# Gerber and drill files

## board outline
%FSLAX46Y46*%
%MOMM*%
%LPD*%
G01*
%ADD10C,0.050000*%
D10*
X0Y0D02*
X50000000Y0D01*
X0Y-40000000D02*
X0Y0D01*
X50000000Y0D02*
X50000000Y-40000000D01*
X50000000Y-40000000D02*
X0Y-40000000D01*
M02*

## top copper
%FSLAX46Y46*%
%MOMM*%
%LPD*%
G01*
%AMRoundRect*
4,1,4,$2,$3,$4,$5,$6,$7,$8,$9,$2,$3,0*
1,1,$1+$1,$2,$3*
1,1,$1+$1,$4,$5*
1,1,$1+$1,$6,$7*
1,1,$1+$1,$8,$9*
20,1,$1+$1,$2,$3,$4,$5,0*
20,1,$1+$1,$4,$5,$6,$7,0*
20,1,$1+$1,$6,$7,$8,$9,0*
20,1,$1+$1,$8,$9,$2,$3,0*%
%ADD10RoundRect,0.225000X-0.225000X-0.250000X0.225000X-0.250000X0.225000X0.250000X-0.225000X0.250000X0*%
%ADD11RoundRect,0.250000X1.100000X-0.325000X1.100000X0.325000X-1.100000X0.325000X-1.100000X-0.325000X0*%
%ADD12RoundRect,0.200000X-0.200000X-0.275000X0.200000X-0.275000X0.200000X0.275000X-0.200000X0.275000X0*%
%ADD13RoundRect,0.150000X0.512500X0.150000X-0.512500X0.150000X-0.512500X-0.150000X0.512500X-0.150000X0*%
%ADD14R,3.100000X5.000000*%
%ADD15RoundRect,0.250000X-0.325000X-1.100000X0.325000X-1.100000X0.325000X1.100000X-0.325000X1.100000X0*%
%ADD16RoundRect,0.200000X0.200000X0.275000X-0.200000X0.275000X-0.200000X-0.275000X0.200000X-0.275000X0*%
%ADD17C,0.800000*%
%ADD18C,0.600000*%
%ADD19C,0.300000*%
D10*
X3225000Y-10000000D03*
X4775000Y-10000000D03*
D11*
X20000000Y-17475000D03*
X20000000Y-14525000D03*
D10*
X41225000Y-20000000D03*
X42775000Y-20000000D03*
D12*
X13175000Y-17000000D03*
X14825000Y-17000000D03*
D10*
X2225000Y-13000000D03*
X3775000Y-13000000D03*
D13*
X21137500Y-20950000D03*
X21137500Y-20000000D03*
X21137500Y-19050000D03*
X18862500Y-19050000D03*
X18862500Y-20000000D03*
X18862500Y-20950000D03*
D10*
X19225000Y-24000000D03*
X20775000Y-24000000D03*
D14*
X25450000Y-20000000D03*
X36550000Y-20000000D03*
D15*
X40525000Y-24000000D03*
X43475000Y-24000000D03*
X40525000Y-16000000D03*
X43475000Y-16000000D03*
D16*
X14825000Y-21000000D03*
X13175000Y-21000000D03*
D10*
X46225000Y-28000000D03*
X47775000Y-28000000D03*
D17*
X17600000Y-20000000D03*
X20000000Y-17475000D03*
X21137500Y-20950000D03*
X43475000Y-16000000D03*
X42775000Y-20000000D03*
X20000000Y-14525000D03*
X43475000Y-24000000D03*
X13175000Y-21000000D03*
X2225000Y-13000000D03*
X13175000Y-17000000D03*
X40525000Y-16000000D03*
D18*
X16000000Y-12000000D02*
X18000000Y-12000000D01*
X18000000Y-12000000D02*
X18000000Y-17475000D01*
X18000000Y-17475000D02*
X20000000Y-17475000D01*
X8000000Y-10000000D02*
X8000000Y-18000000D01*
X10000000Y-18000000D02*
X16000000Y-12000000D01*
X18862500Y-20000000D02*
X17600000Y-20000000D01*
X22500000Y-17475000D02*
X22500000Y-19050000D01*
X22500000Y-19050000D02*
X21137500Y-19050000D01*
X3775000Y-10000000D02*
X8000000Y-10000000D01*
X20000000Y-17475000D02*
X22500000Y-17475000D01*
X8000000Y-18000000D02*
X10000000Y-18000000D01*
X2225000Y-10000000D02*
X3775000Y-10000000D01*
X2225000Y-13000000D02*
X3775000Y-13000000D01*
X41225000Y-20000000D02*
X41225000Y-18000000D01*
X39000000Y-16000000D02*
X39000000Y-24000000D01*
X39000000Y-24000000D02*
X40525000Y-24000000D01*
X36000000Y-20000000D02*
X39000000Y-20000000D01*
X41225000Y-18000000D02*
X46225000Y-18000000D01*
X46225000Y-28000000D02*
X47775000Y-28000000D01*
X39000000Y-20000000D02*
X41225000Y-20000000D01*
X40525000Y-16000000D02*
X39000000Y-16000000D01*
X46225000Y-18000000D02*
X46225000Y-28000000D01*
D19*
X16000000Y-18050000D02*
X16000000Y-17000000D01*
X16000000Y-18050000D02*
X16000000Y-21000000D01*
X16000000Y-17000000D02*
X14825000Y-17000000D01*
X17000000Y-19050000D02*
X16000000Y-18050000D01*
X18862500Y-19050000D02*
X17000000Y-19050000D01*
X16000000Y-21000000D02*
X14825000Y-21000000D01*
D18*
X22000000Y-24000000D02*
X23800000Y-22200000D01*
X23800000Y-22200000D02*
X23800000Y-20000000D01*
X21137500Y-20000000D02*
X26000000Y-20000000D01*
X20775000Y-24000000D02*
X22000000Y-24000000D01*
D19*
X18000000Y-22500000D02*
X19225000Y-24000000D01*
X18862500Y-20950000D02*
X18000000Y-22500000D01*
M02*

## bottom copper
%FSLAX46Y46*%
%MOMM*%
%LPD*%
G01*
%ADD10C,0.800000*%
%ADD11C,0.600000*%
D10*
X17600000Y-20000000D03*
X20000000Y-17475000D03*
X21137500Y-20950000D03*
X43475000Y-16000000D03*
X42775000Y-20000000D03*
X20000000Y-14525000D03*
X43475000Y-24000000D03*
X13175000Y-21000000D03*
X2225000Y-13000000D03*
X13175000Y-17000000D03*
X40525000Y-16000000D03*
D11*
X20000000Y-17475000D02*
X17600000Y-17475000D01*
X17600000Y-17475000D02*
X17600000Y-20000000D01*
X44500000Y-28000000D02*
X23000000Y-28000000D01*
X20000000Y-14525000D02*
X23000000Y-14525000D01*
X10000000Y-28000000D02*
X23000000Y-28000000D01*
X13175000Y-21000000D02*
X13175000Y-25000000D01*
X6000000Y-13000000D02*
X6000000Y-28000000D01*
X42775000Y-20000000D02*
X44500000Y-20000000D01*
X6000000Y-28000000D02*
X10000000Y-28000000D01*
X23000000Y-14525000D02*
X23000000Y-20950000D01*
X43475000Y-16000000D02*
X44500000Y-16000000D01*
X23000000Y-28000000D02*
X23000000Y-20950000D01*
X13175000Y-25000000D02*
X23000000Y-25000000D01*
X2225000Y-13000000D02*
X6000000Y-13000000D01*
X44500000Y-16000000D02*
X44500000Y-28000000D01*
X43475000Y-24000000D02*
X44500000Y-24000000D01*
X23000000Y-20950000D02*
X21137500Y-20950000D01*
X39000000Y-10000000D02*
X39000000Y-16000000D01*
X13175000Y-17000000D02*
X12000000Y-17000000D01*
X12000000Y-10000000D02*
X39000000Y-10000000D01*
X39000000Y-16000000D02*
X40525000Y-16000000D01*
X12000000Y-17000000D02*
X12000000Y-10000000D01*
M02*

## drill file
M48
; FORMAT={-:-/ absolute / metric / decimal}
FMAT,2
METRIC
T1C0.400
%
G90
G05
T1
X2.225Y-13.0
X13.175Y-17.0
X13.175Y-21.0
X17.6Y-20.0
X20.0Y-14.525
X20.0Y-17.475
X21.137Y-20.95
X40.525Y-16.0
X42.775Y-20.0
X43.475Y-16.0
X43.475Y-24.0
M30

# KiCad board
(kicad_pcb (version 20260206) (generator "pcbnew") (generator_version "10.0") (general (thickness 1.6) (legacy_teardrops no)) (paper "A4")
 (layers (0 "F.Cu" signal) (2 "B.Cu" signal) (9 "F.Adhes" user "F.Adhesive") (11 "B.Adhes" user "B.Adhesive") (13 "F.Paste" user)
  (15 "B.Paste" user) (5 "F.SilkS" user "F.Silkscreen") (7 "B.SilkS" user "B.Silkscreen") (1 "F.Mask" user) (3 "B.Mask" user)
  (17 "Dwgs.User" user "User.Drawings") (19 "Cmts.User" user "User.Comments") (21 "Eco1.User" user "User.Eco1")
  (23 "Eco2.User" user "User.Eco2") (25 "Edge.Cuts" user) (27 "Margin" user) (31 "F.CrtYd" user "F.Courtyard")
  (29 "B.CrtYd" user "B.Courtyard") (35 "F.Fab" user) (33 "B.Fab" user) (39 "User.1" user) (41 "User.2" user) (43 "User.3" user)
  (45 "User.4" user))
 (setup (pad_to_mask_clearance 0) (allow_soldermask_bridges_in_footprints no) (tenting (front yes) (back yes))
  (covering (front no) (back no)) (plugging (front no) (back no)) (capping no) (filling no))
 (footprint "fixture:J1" (layer "F.Cu") (at 4 10)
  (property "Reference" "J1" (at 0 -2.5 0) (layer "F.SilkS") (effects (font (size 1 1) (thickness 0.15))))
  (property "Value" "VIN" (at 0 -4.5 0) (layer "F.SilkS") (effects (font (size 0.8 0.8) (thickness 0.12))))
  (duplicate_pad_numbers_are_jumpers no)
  (pad "1" smd roundrect (at -0.775 0) (size 0.9 0.95) (layers "F.Cu" "F.Mask" "F.Paste") (roundrect_rratio 0.25) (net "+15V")
   (thermal_bridge_angle 45))
  (pad "2" smd roundrect (at 0.775 0) (size 0.9 0.95) (layers "F.Cu" "F.Mask" "F.Paste") (roundrect_rratio 0.25) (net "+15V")
   (thermal_bridge_angle 45)))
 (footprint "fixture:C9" (layer "F.Cu") (at 20 16 90)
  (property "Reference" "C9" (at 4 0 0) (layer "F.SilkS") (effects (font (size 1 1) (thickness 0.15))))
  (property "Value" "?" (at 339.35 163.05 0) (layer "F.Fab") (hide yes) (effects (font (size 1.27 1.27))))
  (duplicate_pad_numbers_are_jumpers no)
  (pad "1" smd roundrect (at -1.475 0 90) (size 1.15 2.7) (layers "F.Cu" "F.Mask" "F.Paste") (roundrect_rratio 0.217391) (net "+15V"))
  (pad "2" smd roundrect (at 1.475 0 90) (size 1.15 2.7) (layers "F.Cu" "F.Mask" "F.Paste") (roundrect_rratio 0.217391) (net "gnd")))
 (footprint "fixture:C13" (layer "F.Cu") (at 42 20)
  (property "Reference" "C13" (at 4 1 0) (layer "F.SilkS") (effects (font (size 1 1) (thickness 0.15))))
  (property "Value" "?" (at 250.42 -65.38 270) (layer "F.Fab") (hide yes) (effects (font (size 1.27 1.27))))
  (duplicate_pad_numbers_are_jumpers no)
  (pad "1" smd roundrect (at -0.775 0) (size 0.9 0.95) (layers "F.Cu" "F.Mask" "F.Paste") (roundrect_rratio 0.25) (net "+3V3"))
  (pad "2" smd roundrect (at 0.775 0) (size 0.9 0.95) (layers "F.Cu" "F.Mask" "F.Paste") (roundrect_rratio 0.25) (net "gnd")))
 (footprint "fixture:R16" (layer "F.Cu") (at 14 17)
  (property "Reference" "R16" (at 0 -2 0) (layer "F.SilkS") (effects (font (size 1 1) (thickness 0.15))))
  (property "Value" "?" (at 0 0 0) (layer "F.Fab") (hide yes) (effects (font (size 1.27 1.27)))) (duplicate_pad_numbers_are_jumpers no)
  (pad "1" smd roundrect (at -0.825 0) (size 0.8 0.95) (layers "F.Cu" "F.Mask" "F.Paste") (roundrect_rratio 0.25) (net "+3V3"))
  (pad "2" smd roundrect (at 0.825 0) (size 0.8 0.95) (layers "F.Cu" "F.Mask" "F.Paste") (roundrect_rratio 0.25) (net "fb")))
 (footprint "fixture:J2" (layer "F.Cu") (at 3 13)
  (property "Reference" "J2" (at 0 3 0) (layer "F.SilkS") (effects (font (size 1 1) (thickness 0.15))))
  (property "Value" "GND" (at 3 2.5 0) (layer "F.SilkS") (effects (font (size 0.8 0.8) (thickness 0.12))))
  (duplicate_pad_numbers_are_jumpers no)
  (pad "1" smd roundrect (at -0.775 0) (size 0.9 0.95) (layers "F.Cu" "F.Mask" "F.Paste") (roundrect_rratio 0.25) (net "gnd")
   (thermal_bridge_angle 45))
  (pad "2" smd roundrect (at 0.775 0) (size 0.9 0.95) (layers "F.Cu" "F.Mask" "F.Paste") (roundrect_rratio 0.25) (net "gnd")
   (thermal_bridge_angle 45)))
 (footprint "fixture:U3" (layer "F.Cu") (at 20 20 180)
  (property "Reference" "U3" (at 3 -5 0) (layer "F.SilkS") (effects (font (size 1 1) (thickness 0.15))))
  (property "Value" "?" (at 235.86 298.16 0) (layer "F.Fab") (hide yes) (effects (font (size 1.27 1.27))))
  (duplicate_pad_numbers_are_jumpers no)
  (pad "1" smd roundrect (at -1.1375 -0.95 180) (size 1.325 0.6) (layers "F.Cu" "F.Mask" "F.Paste") (roundrect_rratio 0.25) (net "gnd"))
  (pad "2" smd roundrect (at -1.1375 0 180) (size 1.325 0.6) (layers "F.Cu" "F.Mask" "F.Paste") (roundrect_rratio 0.25) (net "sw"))
  (pad "3" smd roundrect (at -1.1375 0.95 180) (size 1.325 0.6) (layers "F.Cu" "F.Mask" "F.Paste") (roundrect_rratio 0.25) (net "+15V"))
  (pad "4" smd roundrect (at 1.1375 0.95 180) (size 1.325 0.6) (layers "F.Cu" "F.Mask" "F.Paste") (roundrect_rratio 0.25) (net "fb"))
  (pad "5" smd roundrect (at 1.1375 0 180) (size 1.325 0.6) (layers "F.Cu" "F.Mask" "F.Paste") (roundrect_rratio 0.25) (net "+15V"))
  (pad "6" smd roundrect (at 1.1375 -0.95 180) (size 1.325 0.6) (layers "F.Cu" "F.Mask" "F.Paste") (roundrect_rratio 0.25) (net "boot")))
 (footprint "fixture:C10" (layer "F.Cu") (at 20 24)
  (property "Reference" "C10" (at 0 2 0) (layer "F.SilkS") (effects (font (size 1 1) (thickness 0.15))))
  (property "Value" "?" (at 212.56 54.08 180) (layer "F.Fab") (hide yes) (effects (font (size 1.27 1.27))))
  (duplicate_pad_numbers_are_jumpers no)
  (pad "1" smd roundrect (at -0.775 0) (size 0.9 0.95) (layers "F.Cu" "F.Mask" "F.Paste") (roundrect_rratio 0.25) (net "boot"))
  (pad "2" smd roundrect (at 0.775 0) (size 0.9 0.95) (layers "F.Cu" "F.Mask" "F.Paste") (roundrect_rratio 0.25) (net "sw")))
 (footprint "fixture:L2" (layer "F.Cu") (at 31 20)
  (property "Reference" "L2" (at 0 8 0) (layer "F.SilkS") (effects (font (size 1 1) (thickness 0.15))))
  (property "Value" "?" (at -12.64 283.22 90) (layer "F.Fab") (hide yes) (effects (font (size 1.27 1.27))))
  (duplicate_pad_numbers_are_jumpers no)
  (pad "1" smd rect (at -5.55 0) (size 3.1 5) (layers "F.Cu" "F.Mask" "F.Paste") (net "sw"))
  (pad "2" smd rect (at 5.55 0) (size 3.1 5) (layers "F.Cu" "F.Mask" "F.Paste") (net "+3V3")))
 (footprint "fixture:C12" (layer "F.Cu") (at 42 24)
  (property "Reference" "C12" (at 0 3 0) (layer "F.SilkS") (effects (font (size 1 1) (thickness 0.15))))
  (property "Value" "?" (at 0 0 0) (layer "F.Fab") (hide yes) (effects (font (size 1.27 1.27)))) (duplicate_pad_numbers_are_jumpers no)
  (pad "1" smd roundrect (at -1.475 0) (size 1.15 2.7) (layers "F.Cu" "F.Mask" "F.Paste") (roundrect_rratio 0.217391) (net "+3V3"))
  (pad "2" smd roundrect (at 1.475 0) (size 1.15 2.7) (layers "F.Cu" "F.Mask" "F.Paste") (roundrect_rratio 0.217391) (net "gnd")))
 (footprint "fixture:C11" (layer "F.Cu") (at 42 16)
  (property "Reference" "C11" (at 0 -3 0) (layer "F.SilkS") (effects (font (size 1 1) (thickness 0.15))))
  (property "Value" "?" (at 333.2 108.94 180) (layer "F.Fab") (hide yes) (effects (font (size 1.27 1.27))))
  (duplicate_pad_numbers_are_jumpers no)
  (pad "1" smd roundrect (at -1.475 0) (size 1.15 2.7) (layers "F.Cu" "F.Mask" "F.Paste") (roundrect_rratio 0.217391) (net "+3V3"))
  (pad "2" smd roundrect (at 1.475 0) (size 1.15 2.7) (layers "F.Cu" "F.Mask" "F.Paste") (roundrect_rratio 0.217391) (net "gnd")))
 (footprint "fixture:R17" (layer "F.Cu") (at 14 21 180)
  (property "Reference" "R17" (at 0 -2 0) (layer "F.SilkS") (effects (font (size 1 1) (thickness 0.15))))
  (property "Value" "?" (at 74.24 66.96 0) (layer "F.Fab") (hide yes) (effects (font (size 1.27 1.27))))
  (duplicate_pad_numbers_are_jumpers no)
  (pad "1" smd roundrect (at -0.825 0 180) (size 0.8 0.95) (layers "F.Cu" "F.Mask" "F.Paste") (roundrect_rratio 0.25) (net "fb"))
  (pad "2" smd roundrect (at 0.825 0 180) (size 0.8 0.95) (layers "F.Cu" "F.Mask" "F.Paste") (roundrect_rratio 0.25) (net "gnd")))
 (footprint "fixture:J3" (layer "F.Cu") (at 47 28)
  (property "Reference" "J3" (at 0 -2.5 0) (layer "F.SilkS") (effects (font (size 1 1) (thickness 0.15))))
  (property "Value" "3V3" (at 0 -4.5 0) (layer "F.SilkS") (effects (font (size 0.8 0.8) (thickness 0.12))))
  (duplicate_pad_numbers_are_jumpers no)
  (pad "1" smd roundrect (at -0.775 0) (size 0.9 0.95) (layers "F.Cu" "F.Mask" "F.Paste") (roundrect_rratio 0.25) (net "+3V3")
   (thermal_bridge_angle 45))
  (pad "2" smd roundrect (at 0.775 0) (size 0.9 0.95) (layers "F.Cu" "F.Mask" "F.Paste") (roundrect_rratio 0.25) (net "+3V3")
   (thermal_bridge_angle 45)))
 (gr_line (start 0 0) (end 50 0) (stroke (width 0.05) (type default)) (layer "Edge.Cuts"))
 (gr_line (start 0 40) (end 0 0) (stroke (width 0.05) (type default)) (layer "Edge.Cuts"))
 (gr_line (start 50 0) (end 50 40) (stroke (width 0.05) (type default)) (layer "Edge.Cuts"))
 (gr_line (start 50 40) (end 0 40) (stroke (width 0.05) (type default)) (layer "Edge.Cuts"))
 (segment (start 16 12) (end 18 12) (width 0.6) (layer "F.Cu") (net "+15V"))
 (segment (start 18 12) (end 18 17.475) (width 0.6) (layer "F.Cu") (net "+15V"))
 (segment (start 18 17.475) (end 20 17.475) (width 0.6) (layer "F.Cu") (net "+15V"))
 (segment (start 8 10) (end 8 18) (width 0.6) (layer "F.Cu") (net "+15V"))
 (segment (start 10 18) (end 16 12) (width 0.6) (layer "F.Cu") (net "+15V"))
 (segment (start 18.8625 20) (end 17.6 20) (width 0.6) (layer "F.Cu") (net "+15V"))
 (segment (start 22.5 17.475) (end 22.5 19.05) (width 0.6) (layer "F.Cu") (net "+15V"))
 (segment (start 22.5 19.05) (end 21.1375 19.05) (width 0.6) (layer "F.Cu") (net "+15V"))
 (segment (start 3.775 10) (end 8 10) (width 0.6) (layer "F.Cu") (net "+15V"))
 (segment (start 20 17.475) (end 22.5 17.475) (width 0.6) (layer "F.Cu") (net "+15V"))
 (segment (start 8 18) (end 10 18) (width 0.6) (layer "F.Cu") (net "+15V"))
 (segment (start 2.225 10) (end 3.775 10) (width 0.6) (layer "F.Cu") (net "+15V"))
 (via (at 17.6 20) (size 0.8) (drill 0.4) (layers "F.Cu" "B.Cu") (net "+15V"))
 (via (at 20 17.475) (size 0.8) (drill 0.4) (layers "F.Cu" "B.Cu") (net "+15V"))
 (segment (start 20 17.475) (end 17.6 17.475) (width 0.6) (layer "B.Cu") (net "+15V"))
 (segment (start 17.6 17.475) (end 17.6 20) (width 0.6) (layer "B.Cu") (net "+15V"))
 (segment (start 2.225 13) (end 3.775 13) (width 0.6) (layer "F.Cu") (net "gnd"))
 (via (at 21.1375 20.95) (size 0.8) (drill 0.4) (layers "F.Cu" "B.Cu") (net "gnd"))
 (via (at 43.475 16) (size 0.8) (drill 0.4) (layers "F.Cu" "B.Cu") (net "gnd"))
 (via (at 42.775 20) (size 0.8) (drill 0.4) (layers "F.Cu" "B.Cu") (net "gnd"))
 (via (at 20 14.525) (size 0.8) (drill 0.4) (layers "F.Cu" "B.Cu") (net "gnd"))
 (via (at 43.475 24) (size 0.8) (drill 0.4) (layers "F.Cu" "B.Cu") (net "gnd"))
 (via (at 13.175 21) (size 0.8) (drill 0.4) (layers "F.Cu" "B.Cu") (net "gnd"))
 (via (at 2.225 13) (size 0.8) (drill 0.4) (layers "F.Cu" "B.Cu") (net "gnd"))
 (segment (start 44.5 28) (end 23 28) (width 0.6) (layer "B.Cu") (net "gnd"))
 (segment (start 20 14.525) (end 23 14.525) (width 0.6) (layer "B.Cu") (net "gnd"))
 (segment (start 10 28) (end 23 28) (width 0.6) (layer "B.Cu") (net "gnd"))
 (segment (start 13.175 21) (end 13.175 25) (width 0.6) (layer "B.Cu") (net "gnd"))
 (segment (start 6 13) (end 6 28) (width 0.6) (layer "B.Cu") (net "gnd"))
 (segment (start 42.775 20) (end 44.5 20) (width 0.6) (layer "B.Cu") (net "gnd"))
 (segment (start 6 28) (end 10 28) (width 0.6) (layer "B.Cu") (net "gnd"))
 (segment (start 23 14.525) (end 23 20.95) (width 0.6) (layer "B.Cu") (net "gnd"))
 (segment (start 43.475 16) (end 44.5 16) (width 0.6) (layer "B.Cu") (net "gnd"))
 (segment (start 23 28) (end 23 20.95) (width 0.6) (layer "B.Cu") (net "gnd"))
 (segment (start 13.175 25) (end 23 25) (width 0.6) (layer "B.Cu") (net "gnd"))
 (segment (start 2.225 13) (end 6 13) (width 0.6) (layer "B.Cu") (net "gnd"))
 (segment (start 44.5 16) (end 44.5 28) (width 0.6) (layer "B.Cu") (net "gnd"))
 (segment (start 43.475 24) (end 44.5 24) (width 0.6) (layer "B.Cu") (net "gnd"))
 (segment (start 23 20.95) (end 21.1375 20.95) (width 0.6) (layer "B.Cu") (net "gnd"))
 (segment (start 41.225 20) (end 41.225 18) (width 0.6) (layer "F.Cu") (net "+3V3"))
 (segment (start 39 16) (end 39 24) (width 0.6) (layer "F.Cu") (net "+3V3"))
 (segment (start 39 24) (end 40.525 24) (width 0.6) (layer "F.Cu") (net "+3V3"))
 (segment (start 36 20) (end 39 20) (width 0.6) (layer "F.Cu") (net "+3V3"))
 (segment (start 41.225 18) (end 46.225 18) (width 0.6) (layer "F.Cu") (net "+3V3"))
 (segment (start 46.225 28) (end 47.775 28) (width 0.6) (layer "F.Cu") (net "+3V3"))
 (segment (start 39 20) (end 41.225 20) (width 0.6) (layer "F.Cu") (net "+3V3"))
 (segment (start 40.525 16) (end 39 16) (width 0.6) (layer "F.Cu") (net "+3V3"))
 (segment (start 46.225 18) (end 46.225 28) (width 0.6) (layer "F.Cu") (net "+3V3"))
 (via (at 13.175 17) (size 0.8) (drill 0.4) (layers "F.Cu" "B.Cu") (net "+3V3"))
 (via (at 40.525 16) (size 0.8) (drill 0.4) (layers "F.Cu" "B.Cu") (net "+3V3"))
 (segment (start 39 10) (end 39 16) (width 0.6) (layer "B.Cu") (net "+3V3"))
 (segment (start 13.175 17) (end 12 17) (width 0.6) (layer "B.Cu") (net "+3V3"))
 (segment (start 12 10) (end 39 10) (width 0.6) (layer "B.Cu") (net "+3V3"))
 (segment (start 39 16) (end 40.525 16) (width 0.6) (layer "B.Cu") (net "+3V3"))
 (segment (start 12 17) (end 12 10) (width 0.6) (layer "B.Cu") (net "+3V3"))
 (segment (start 16 18.05) (end 16 17) (width 0.3) (layer "F.Cu") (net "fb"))
 (segment (start 16 18.05) (end 16 21) (width 0.3) (layer "F.Cu") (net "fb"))
 (segment (start 16 17) (end 14.825 17) (width 0.3) (layer "F.Cu") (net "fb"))
 (segment (start 17 19.05) (end 16 18.05) (width 0.3) (layer "F.Cu") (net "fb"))
 (segment (start 18.8625 19.05) (end 17 19.05) (width 0.3) (layer "F.Cu") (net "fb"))
 (segment (start 16 21) (end 14.825 21) (width 0.3) (layer "F.Cu") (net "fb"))
 (segment (start 22 24) (end 23.8 22.2) (width 0.6) (layer "F.Cu") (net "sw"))
 (segment (start 23.8 22.2) (end 23.8 20) (width 0.6) (layer "F.Cu") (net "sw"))
 (segment (start 21.1375 20) (end 26 20) (width 0.6) (layer "F.Cu") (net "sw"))
 (segment (start 20.775 24) (end 22 24) (width 0.6) (layer "F.Cu") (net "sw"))
 (segment (start 18 22.5) (end 19.225 24) (width 0.3) (layer "F.Cu") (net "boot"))
 (segment (start 18.8625 20.95) (end 18 22.5) (width 0.3) (layer "F.Cu") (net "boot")))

